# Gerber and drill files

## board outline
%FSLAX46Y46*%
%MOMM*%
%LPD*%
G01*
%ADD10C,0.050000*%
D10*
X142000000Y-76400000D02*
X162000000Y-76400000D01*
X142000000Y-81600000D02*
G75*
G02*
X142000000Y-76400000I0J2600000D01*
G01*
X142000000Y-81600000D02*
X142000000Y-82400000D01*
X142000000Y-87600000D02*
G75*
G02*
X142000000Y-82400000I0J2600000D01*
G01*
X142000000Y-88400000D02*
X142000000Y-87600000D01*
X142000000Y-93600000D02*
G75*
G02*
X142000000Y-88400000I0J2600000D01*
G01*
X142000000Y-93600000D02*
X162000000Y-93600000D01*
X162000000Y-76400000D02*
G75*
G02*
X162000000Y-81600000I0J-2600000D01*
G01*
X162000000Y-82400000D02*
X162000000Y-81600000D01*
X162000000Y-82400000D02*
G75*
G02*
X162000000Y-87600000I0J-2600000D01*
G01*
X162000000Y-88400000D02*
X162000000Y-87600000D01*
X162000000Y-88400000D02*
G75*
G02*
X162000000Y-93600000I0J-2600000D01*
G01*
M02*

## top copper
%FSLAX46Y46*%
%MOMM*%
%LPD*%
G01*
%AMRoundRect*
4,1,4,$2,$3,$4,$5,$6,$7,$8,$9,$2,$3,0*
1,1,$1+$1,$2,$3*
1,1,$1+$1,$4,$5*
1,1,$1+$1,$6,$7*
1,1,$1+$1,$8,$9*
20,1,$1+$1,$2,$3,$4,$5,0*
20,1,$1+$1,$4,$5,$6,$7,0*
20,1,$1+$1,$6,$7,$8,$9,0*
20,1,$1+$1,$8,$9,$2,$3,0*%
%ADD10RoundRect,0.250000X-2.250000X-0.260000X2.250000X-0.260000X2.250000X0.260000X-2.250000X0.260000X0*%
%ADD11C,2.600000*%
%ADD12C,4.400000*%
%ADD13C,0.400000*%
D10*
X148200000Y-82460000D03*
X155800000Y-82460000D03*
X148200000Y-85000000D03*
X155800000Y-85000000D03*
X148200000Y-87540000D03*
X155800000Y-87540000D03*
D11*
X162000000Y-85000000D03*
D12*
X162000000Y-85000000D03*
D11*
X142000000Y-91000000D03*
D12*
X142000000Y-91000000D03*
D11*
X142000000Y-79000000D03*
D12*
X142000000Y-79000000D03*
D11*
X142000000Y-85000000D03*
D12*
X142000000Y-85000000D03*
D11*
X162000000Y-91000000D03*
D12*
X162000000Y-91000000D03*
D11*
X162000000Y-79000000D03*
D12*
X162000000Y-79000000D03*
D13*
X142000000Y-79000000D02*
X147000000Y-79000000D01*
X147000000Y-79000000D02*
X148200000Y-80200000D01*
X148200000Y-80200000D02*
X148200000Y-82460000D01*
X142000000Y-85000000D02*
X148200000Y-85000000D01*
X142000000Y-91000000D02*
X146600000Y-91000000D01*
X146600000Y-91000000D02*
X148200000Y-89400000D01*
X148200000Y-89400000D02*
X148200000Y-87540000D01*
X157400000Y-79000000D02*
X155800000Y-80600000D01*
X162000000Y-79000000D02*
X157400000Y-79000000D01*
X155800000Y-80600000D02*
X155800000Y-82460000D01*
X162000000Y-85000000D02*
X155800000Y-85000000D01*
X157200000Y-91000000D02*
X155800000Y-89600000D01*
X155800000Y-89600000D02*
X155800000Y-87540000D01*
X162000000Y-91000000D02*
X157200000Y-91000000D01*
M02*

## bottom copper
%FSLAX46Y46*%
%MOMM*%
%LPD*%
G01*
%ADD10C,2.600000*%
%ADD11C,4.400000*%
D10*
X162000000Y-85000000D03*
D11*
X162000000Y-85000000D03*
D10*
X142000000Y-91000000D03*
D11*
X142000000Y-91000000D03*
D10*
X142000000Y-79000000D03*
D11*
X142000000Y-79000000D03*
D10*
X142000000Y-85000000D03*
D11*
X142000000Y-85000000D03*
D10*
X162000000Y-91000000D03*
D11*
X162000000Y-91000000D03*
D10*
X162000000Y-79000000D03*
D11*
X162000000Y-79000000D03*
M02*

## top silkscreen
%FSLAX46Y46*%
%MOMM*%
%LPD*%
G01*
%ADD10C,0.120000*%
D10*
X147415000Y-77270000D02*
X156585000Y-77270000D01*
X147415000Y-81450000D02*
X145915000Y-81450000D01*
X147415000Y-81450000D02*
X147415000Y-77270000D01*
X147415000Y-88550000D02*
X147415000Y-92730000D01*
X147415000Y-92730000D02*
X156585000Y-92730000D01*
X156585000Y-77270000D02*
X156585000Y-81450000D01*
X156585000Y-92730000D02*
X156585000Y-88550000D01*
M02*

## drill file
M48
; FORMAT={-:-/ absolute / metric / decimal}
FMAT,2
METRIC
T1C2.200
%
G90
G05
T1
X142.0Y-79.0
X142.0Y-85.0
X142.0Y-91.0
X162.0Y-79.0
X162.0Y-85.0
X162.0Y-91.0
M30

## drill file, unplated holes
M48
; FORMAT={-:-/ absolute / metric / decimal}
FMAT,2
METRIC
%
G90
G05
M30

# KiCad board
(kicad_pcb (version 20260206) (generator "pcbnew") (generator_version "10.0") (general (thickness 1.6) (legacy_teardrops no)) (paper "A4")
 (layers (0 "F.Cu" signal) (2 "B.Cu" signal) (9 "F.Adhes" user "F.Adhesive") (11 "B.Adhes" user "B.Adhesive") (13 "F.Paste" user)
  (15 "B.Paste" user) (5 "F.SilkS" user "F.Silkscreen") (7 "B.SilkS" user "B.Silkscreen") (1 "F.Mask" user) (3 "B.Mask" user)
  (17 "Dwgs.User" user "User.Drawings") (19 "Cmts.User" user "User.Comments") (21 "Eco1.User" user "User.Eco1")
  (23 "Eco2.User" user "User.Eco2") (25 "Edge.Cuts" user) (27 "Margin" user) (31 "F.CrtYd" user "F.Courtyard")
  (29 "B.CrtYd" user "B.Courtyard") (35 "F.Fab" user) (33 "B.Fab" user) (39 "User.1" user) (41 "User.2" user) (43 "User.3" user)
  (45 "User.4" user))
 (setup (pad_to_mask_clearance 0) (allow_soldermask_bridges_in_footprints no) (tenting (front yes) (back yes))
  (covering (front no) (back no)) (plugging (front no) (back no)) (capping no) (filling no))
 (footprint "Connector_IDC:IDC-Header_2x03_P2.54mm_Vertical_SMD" (layer "F.Cu") (at 152 85)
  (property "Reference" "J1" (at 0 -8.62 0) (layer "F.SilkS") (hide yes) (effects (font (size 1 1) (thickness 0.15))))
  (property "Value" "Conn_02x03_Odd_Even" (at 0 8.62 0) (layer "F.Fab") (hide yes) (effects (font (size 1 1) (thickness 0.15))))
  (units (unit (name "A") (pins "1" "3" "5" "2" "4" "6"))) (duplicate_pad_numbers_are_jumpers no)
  (fp_line (start -4.585 -7.73) (end 4.585 -7.73) (stroke (width 0.12) (type solid)) (layer "F.SilkS"))
  (fp_line (start -4.585 -3.55) (end -6.085 -3.55) (stroke (width 0.12) (type solid)) (layer "F.SilkS"))
  (fp_line (start -4.585 -3.55) (end -4.585 -7.73) (stroke (width 0.12) (type solid)) (layer "F.SilkS"))
  (fp_line (start -4.585 3.55) (end -4.585 7.73) (stroke (width 0.12) (type solid)) (layer "F.SilkS"))
  (fp_line (start -4.585 7.73) (end 4.585 7.73) (stroke (width 0.12) (type solid)) (layer "F.SilkS"))
  (fp_line (start 4.585 -7.73) (end 4.585 -3.55) (stroke (width 0.12) (type solid)) (layer "F.SilkS"))
  (fp_line (start 4.585 7.73) (end 4.585 3.55) (stroke (width 0.12) (type solid)) (layer "F.SilkS"))
  (pad "1" smd roundrect (at -3.8 -2.54) (size 5 1.02) (layers "F.Cu" "F.Mask" "F.Paste") (roundrect_rratio 0.245098) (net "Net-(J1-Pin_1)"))
  (pad "2" smd roundrect (at 3.8 -2.54) (size 5 1.02) (layers "F.Cu" "F.Mask" "F.Paste") (roundrect_rratio 0.245098) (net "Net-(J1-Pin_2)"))
  (pad "3" smd roundrect (at -3.8 0) (size 5 1.02) (layers "F.Cu" "F.Mask" "F.Paste") (roundrect_rratio 0.245098) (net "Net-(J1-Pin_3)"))
  (pad "4" smd roundrect (at 3.8 0) (size 5 1.02) (layers "F.Cu" "F.Mask" "F.Paste") (roundrect_rratio 0.245098) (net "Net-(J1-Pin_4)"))
  (pad "5" smd roundrect (at -3.8 2.54) (size 5 1.02) (layers "F.Cu" "F.Mask" "F.Paste") (roundrect_rratio 0.245098) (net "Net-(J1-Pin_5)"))
  (pad "6" smd roundrect (at 3.8 2.54) (size 5 1.02) (layers "F.Cu" "F.Mask" "F.Paste") (roundrect_rratio 0.245098) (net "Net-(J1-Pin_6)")))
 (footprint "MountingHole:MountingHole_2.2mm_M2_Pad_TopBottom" (layer "F.Cu") (at 162 85)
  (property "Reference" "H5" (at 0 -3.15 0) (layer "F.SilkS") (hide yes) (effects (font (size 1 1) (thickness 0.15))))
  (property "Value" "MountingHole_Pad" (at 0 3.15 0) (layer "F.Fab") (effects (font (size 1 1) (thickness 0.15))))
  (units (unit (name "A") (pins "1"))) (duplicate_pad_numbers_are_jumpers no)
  (pad "1" thru_hole circle (at 0 0) (size 2.6 2.6) (drill 2.2) (layers "*.Cu" "*.Mask") (remove_unused_layers no) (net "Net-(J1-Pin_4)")
   (zone_connect 2))
  (pad "1" connect circle (at 0 0) (size 4.4 4.4) (layers "F.Cu" "F.Mask") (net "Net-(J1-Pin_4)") (zone_connect 2))
  (pad "1" connect circle (at 0 0) (size 4.4 4.4) (layers "B.Cu" "B.Mask") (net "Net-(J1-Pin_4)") (zone_connect 2)))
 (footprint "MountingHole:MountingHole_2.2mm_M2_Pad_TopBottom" (layer "F.Cu") (at 142 91)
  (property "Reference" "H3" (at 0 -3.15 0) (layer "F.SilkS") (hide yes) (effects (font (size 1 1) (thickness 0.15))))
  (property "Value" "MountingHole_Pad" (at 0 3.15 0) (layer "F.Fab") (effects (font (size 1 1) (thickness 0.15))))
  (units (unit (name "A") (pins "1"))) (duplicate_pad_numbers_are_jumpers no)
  (pad "1" thru_hole circle (at 0 0) (size 2.6 2.6) (drill 2.2) (layers "*.Cu" "*.Mask") (remove_unused_layers no) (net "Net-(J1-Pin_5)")
   (zone_connect 2))
  (pad "1" connect circle (at 0 0) (size 4.4 4.4) (layers "F.Cu" "F.Mask") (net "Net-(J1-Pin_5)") (zone_connect 2))
  (pad "1" connect circle (at 0 0) (size 4.4 4.4) (layers "B.Cu" "B.Mask") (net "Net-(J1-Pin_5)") (zone_connect 2)))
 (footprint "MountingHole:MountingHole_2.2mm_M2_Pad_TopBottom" (layer "F.Cu") (at 142 79)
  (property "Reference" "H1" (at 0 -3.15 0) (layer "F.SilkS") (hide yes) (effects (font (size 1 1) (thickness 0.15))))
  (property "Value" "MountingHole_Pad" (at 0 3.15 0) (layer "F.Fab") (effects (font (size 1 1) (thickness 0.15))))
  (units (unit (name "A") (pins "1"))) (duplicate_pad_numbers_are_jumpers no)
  (pad "1" thru_hole circle (at 0 0) (size 2.6 2.6) (drill 2.2) (layers "*.Cu" "*.Mask") (remove_unused_layers no) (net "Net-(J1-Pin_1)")
   (zone_connect 2))
  (pad "1" connect circle (at 0 0) (size 4.4 4.4) (layers "F.Cu" "F.Mask") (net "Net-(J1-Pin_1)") (zone_connect 2))
  (pad "1" connect circle (at 0 0) (size 4.4 4.4) (layers "B.Cu" "B.Mask") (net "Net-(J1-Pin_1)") (zone_connect 2)))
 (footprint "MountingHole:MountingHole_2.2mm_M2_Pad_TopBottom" (layer "F.Cu") (at 142 85)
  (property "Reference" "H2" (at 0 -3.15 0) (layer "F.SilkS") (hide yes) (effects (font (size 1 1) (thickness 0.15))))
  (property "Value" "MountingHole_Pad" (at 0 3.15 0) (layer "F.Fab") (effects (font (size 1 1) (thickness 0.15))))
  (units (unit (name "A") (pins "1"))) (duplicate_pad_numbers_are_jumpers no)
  (pad "1" thru_hole circle (at 0 0) (size 2.6 2.6) (drill 2.2) (layers "*.Cu" "*.Mask") (remove_unused_layers no) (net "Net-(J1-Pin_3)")
   (zone_connect 2))
  (pad "1" connect circle (at 0 0) (size 4.4 4.4) (layers "F.Cu" "F.Mask") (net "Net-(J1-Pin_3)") (zone_connect 2))
  (pad "1" connect circle (at 0 0) (size 4.4 4.4) (layers "B.Cu" "B.Mask") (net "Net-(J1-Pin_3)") (zone_connect 2)))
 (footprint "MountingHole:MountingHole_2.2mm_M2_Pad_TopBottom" (layer "F.Cu") (at 162 91)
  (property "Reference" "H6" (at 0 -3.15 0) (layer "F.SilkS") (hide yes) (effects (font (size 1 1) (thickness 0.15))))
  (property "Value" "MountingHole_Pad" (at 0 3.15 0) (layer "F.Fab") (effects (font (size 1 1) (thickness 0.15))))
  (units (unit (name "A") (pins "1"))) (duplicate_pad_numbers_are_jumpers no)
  (pad "1" thru_hole circle (at 0 0) (size 2.6 2.6) (drill 2.2) (layers "*.Cu" "*.Mask") (remove_unused_layers no) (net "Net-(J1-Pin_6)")
   (zone_connect 2))
  (pad "1" connect circle (at 0 0) (size 4.4 4.4) (layers "F.Cu" "F.Mask") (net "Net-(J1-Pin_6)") (zone_connect 2))
  (pad "1" connect circle (at 0 0) (size 4.4 4.4) (layers "B.Cu" "B.Mask") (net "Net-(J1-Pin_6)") (zone_connect 2)))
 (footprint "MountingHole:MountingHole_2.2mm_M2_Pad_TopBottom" (layer "F.Cu") (at 162 79)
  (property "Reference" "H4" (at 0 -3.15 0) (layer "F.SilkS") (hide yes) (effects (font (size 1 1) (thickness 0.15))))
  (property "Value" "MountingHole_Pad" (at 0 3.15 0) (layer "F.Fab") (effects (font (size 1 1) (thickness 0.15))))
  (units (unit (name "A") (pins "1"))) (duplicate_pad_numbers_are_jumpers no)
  (pad "1" thru_hole circle (at 0 0) (size 2.6 2.6) (drill 2.2) (layers "*.Cu" "*.Mask") (remove_unused_layers no) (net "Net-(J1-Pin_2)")
   (zone_connect 2))
  (pad "1" connect circle (at 0 0) (size 4.4 4.4) (layers "F.Cu" "F.Mask") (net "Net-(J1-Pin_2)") (zone_connect 2))
  (pad "1" connect circle (at 0 0) (size 4.4 4.4) (layers "B.Cu" "B.Mask") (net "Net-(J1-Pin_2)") (zone_connect 2)))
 (gr_line (start 142 76.4) (end 162 76.4) (stroke (width 0.05) (type default)) (layer "Edge.Cuts"))
 (gr_arc (start 142 81.6) (mid 139.4 79) (end 142 76.4) (stroke (width 0.05) (type default)) (layer "Edge.Cuts"))
 (gr_line (start 142 81.6) (end 142 82.4) (stroke (width 0.05) (type default)) (layer "Edge.Cuts"))
 (gr_arc (start 142 87.6) (mid 139.4 85) (end 142 82.4) (stroke (width 0.05) (type default)) (layer "Edge.Cuts"))
 (gr_line (start 142 88.4) (end 142 87.6) (stroke (width 0.05) (type default)) (layer "Edge.Cuts"))
 (gr_arc (start 142 93.6) (mid 139.4 91) (end 142 88.4) (stroke (width 0.05) (type default)) (layer "Edge.Cuts"))
 (gr_line (start 142 93.6) (end 162 93.6) (stroke (width 0.05) (type default)) (layer "Edge.Cuts"))
 (gr_arc (start 162 76.4) (mid 164.6 79) (end 162 81.6) (stroke (width 0.05) (type default)) (layer "Edge.Cuts"))
 (gr_line (start 162 82.4) (end 162 81.6) (stroke (width 0.05) (type default)) (layer "Edge.Cuts"))
 (gr_arc (start 162 82.4) (mid 164.6 85) (end 162 87.6) (stroke (width 0.05) (type default)) (layer "Edge.Cuts"))
 (gr_line (start 162 88.4) (end 162 87.6) (stroke (width 0.05) (type default)) (layer "Edge.Cuts"))
 (gr_arc (start 162 88.4) (mid 164.6 91) (end 162 93.6) (stroke (width 0.05) (type default)) (layer "Edge.Cuts"))
 (segment (start 142 79) (end 147 79) (width 0.4) (layer "F.Cu") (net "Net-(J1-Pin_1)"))
 (segment (start 147 79) (end 148.2 80.2) (width 0.4) (layer "F.Cu") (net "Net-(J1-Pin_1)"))
 (segment (start 148.2 80.2) (end 148.2 82.46) (width 0.4) (layer "F.Cu") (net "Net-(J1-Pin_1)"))
 (segment (start 157.4 79) (end 155.8 80.6) (width 0.4) (layer "F.Cu") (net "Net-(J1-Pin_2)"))
 (segment (start 162 79) (end 157.4 79) (width 0.4) (layer "F.Cu") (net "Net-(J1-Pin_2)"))
 (segment (start 155.8 80.6) (end 155.8 82.46) (width 0.4) (layer "F.Cu") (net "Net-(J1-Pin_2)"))
 (segment (start 142 85) (end 148.2 85) (width 0.4) (layer "F.Cu") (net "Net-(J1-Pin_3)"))
 (segment (start 162 85) (end 155.8 85) (width 0.4) (layer "F.Cu") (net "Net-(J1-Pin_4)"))
 (segment (start 142 91) (end 146.6 91) (width 0.4) (layer "F.Cu") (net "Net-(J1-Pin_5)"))
 (segment (start 146.6 91) (end 148.2 89.4) (width 0.4) (layer "F.Cu") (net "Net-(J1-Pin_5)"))
 (segment (start 148.2 89.4) (end 148.2 87.54) (width 0.4) (layer "F.Cu") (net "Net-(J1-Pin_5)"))
 (segment (start 157.2 91) (end 155.8 89.6) (width 0.4) (layer "F.Cu") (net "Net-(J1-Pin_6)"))
 (segment (start 155.8 89.6) (end 155.8 87.54) (width 0.4) (layer "F.Cu") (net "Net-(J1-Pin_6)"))
 (segment (start 162 91) (end 157.2 91) (width 0.4) (layer "F.Cu") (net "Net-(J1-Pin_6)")))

